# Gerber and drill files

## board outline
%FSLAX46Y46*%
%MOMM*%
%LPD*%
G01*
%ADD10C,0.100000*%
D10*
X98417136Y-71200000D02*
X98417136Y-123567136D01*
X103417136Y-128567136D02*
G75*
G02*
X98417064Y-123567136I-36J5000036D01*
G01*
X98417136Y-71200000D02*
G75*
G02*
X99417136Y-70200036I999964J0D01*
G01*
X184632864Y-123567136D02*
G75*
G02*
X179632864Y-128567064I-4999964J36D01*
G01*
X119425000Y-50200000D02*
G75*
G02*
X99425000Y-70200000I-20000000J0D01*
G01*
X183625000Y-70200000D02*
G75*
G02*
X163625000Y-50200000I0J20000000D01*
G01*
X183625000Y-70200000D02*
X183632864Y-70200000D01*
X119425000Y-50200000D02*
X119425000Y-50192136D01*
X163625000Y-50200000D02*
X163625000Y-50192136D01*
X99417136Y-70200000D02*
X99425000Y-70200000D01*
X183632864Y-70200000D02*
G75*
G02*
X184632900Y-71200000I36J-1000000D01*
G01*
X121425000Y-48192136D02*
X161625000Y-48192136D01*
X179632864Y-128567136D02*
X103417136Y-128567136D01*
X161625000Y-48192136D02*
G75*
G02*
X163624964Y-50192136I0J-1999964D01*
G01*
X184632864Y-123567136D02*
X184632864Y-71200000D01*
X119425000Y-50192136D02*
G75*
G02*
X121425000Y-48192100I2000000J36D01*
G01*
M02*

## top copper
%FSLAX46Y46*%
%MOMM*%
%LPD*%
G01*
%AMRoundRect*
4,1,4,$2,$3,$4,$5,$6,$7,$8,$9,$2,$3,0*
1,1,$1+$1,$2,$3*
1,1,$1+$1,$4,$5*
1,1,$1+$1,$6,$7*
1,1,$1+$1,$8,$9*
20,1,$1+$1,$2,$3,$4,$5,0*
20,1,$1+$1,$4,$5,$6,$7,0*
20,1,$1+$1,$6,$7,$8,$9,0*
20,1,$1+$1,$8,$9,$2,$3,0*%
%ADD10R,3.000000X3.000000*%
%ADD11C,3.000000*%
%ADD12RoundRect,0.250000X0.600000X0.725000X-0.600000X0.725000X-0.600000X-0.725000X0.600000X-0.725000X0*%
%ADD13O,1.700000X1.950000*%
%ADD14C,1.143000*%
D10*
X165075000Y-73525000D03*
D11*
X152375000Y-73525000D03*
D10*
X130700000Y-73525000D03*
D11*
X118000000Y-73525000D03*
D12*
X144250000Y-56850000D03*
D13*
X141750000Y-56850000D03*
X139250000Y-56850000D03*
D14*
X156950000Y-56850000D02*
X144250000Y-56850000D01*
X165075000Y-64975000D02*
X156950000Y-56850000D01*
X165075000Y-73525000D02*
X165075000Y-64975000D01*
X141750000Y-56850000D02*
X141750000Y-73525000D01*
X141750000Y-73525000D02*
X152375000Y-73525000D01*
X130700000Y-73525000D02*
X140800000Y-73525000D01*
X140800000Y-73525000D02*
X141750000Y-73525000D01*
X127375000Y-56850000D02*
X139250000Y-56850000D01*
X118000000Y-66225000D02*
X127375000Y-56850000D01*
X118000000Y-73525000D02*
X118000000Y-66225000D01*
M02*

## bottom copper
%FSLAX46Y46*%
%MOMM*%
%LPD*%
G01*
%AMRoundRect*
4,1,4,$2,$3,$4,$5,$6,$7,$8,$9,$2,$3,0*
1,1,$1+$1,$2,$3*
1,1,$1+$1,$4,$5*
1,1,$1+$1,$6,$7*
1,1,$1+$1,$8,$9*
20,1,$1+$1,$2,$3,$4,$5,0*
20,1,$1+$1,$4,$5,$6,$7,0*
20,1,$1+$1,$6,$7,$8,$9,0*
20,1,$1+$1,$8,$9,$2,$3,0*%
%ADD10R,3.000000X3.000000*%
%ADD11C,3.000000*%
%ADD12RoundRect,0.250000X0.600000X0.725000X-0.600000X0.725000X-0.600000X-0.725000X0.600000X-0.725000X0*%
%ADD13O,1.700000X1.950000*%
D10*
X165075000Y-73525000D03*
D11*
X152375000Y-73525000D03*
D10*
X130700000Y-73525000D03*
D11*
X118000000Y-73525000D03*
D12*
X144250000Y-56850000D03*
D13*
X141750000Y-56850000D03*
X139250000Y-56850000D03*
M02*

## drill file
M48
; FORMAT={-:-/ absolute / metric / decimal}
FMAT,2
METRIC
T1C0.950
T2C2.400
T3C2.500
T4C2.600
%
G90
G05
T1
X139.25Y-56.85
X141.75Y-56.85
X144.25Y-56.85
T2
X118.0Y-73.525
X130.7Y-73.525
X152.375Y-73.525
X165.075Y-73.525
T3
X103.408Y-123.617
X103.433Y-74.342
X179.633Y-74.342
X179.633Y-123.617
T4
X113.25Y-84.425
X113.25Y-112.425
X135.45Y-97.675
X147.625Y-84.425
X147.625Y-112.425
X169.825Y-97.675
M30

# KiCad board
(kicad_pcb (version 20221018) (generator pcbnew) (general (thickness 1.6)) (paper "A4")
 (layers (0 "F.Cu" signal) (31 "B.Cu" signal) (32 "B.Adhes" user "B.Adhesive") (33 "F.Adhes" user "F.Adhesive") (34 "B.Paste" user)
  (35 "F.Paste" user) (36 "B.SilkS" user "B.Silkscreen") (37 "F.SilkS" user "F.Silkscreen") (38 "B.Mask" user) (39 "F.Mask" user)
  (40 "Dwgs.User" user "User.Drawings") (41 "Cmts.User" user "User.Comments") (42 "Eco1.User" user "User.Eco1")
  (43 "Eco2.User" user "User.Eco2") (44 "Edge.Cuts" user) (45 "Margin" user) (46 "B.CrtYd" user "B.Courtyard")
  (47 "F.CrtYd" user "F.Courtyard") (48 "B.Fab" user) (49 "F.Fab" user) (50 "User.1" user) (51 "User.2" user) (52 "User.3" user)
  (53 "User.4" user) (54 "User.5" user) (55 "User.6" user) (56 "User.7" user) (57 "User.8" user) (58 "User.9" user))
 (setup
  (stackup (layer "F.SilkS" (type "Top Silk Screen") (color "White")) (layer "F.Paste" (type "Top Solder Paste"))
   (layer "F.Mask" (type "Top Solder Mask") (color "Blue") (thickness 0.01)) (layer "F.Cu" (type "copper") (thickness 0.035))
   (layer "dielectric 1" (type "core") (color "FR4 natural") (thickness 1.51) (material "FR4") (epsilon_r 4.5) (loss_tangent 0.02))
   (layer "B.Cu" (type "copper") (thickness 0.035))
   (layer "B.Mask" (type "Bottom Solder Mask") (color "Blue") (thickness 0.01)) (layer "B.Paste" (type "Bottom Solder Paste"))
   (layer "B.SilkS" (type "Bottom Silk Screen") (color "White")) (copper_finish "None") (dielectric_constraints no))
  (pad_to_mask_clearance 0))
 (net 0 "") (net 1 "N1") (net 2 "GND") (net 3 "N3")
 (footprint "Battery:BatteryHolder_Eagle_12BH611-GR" (layer "F.Cu") (at 165.075 73.525 90)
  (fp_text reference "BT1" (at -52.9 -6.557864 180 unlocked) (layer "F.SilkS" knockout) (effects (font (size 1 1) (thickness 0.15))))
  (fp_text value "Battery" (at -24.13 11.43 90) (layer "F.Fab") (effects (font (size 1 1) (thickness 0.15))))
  (pad "" np_thru_hole circle (at -38.9 -17.45 90) (size 2.6 2.6) (drill 2.6) (layers "*.Cu" "*.Mask"))
  (pad "" np_thru_hole circle (at -24.15 4.75 90) (size 2.6 2.6) (drill 2.6) (layers "*.Cu" "*.Mask"))
  (pad "" np_thru_hole circle (at -10.9 -17.45 90) (size 2.6 2.6) (drill 2.6) (layers "*.Cu" "*.Mask"))
  (pad "1" thru_hole rect (at 0 0 90) (size 3 3) (drill 2.4) (layers "*.Cu" "*.Mask") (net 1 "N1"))
  (pad "2" thru_hole circle (at 0 -12.7 90) (size 3 3) (drill 2.4) (layers "*.Cu" "*.Mask") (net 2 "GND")))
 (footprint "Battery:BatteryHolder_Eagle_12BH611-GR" (layer "F.Cu") (at 130.7 73.525 90)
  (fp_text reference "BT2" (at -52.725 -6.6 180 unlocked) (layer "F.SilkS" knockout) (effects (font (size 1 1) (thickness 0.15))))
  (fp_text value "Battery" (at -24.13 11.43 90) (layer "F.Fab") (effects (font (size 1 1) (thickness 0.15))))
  (pad "" np_thru_hole circle (at -38.9 -17.45 90) (size 2.6 2.6) (drill 2.6) (layers "*.Cu" "*.Mask"))
  (pad "" np_thru_hole circle (at -24.15 4.75 90) (size 2.6 2.6) (drill 2.6) (layers "*.Cu" "*.Mask"))
  (pad "" np_thru_hole circle (at -10.9 -17.45 90) (size 2.6 2.6) (drill 2.6) (layers "*.Cu" "*.Mask"))
  (pad "1" thru_hole rect (at 0 0 90) (size 3 3) (drill 2.4) (layers "*.Cu" "*.Mask") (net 2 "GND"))
  (pad "2" thru_hole circle (at 0 -12.7 90) (size 3 3) (drill 2.4) (layers "*.Cu" "*.Mask") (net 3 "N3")))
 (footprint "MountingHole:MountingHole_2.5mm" (layer "F.Cu") (at 103.432864 74.342136)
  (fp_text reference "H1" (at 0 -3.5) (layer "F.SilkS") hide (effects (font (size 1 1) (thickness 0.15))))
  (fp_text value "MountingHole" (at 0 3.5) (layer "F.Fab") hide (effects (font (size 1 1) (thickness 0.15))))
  (pad "" np_thru_hole circle (at 0 0) (size 2.5 2.5) (drill 2.5) (layers "*.Cu" "*.Mask")))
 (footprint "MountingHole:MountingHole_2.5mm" (layer "F.Cu") (at 103.407864 123.617136)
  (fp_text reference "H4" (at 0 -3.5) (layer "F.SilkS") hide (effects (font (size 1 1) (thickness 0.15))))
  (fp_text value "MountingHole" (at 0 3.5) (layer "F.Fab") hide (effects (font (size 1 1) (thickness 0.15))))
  (pad "" np_thru_hole circle (at 0 0) (size 2.5 2.5) (drill 2.5) (layers "*.Cu" "*.Mask")))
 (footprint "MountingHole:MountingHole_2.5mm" (layer "F.Cu") (at 179.632864 123.617136)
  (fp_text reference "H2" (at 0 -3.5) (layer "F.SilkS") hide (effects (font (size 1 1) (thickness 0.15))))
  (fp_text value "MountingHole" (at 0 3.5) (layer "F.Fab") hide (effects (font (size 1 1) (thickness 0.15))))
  (pad "" np_thru_hole circle (at 0 0) (size 2.5 2.5) (drill 2.5) (layers "*.Cu" "*.Mask")))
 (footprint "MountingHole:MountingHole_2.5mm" (layer "F.Cu") (at 179.632864 74.342136)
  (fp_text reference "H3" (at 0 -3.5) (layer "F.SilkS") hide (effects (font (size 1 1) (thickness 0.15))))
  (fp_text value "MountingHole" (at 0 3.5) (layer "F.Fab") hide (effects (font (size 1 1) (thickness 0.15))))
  (pad "" np_thru_hole circle (at 0 0) (size 2.5 2.5) (drill 2.5) (layers "*.Cu" "*.Mask")))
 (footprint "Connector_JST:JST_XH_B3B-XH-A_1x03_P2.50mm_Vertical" (layer "B.Cu") (at 144.25 56.85 180)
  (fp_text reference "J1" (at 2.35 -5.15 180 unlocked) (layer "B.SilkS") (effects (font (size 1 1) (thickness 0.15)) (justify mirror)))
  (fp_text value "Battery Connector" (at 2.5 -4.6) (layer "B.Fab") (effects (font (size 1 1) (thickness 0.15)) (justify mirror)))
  (pad "1" thru_hole roundrect (at 0 0 180) (size 1.7 1.95) (drill 0.95) (layers "*.Cu" "*.Mask") (roundrect_rratio 0.1470588235)
   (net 1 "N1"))
  (pad "2" thru_hole oval (at 2.5 0 180) (size 1.7 1.95) (drill 0.95) (layers "*.Cu" "*.Mask") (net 2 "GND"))
  (pad "3" thru_hole oval (at 5 0 180) (size 1.7 1.95) (drill 0.95) (layers "*.Cu" "*.Mask") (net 3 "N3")))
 (gr_line (start 98.417136 71.2) (end 98.417136 123.567136) (stroke (width 0.1) (type default)) (layer "Edge.Cuts"))
 (gr_arc (start 103.417136 128.567136) (mid 99.881602 127.10267) (end 98.417136 123.567136) (stroke (width 0.1) (type default))
  (layer "Edge.Cuts"))
 (gr_arc (start 98.417136 71.2) (mid 98.710029 70.492893) (end 99.417136 70.2) (stroke (width 0.1) (type default)) (layer "Edge.Cuts"))
 (gr_arc (start 184.632864 123.567136) (mid 183.168398 127.10267) (end 179.632864 128.567136) (stroke (width 0.1) (type default))
  (layer "Edge.Cuts"))
 (gr_arc (start 119.425 50.2) (mid 113.567136 64.342136) (end 99.425 70.2) (stroke (width 0.1) (type default)) (layer "Edge.Cuts"))
 (gr_arc (start 183.625 70.2) (mid 169.482864 64.342136) (end 163.625 50.2) (stroke (width 0.1) (type default)) (layer "Edge.Cuts"))
 (gr_line (start 183.625 70.2) (end 183.632864 70.2) (stroke (width 0.1) (type default)) (layer "Edge.Cuts"))
 (gr_line (start 119.425 50.2) (end 119.425 50.192136) (stroke (width 0.1) (type default)) (layer "Edge.Cuts"))
 (gr_line (start 163.625 50.2) (end 163.625 50.192136) (stroke (width 0.1) (type default)) (layer "Edge.Cuts"))
 (gr_line (start 99.417136 70.2) (end 99.425 70.2) (stroke (width 0.1) (type default)) (layer "Edge.Cuts"))
 (gr_arc (start 183.632864 70.2) (mid 184.339971 70.492893) (end 184.632864 71.2) (stroke (width 0.1) (type default)) (layer "Edge.Cuts"))
 (gr_line (start 121.425 48.192136) (end 161.625 48.192136) (stroke (width 0.1) (type default)) (layer "Edge.Cuts"))
 (gr_line (start 179.632864 128.567136) (end 103.417136 128.567136) (stroke (width 0.1) (type default)) (layer "Edge.Cuts"))
 (gr_arc (start 161.625 48.192136) (mid 163.039214 48.777922) (end 163.625 50.192136) (stroke (width 0.1) (type default))
  (layer "Edge.Cuts"))
 (gr_line (start 184.632864 123.567136) (end 184.632864 71.2) (stroke (width 0.1) (type default)) (layer "Edge.Cuts"))
 (gr_arc (start 119.425 50.192136) (mid 120.010786 48.777922) (end 121.425 48.192136) (stroke (width 0.1) (type default))
  (layer "Edge.Cuts"))
 (segment (start 156.95 56.85) (end 144.25 56.85) (width 1.143) (layer "F.Cu") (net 1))
 (segment (start 165.075 64.975) (end 156.95 56.85) (width 1.143) (layer "F.Cu") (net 1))
 (segment (start 165.075 73.525) (end 165.075 64.975) (width 1.143) (layer "F.Cu") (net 1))
 (segment (start 141.75 56.85) (end 141.75 73.525) (width 1.143) (layer "F.Cu") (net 2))
 (segment (start 141.75 73.525) (end 152.375 73.525) (width 1.143) (layer "F.Cu") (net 2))
 (segment (start 130.7 73.525) (end 140.8 73.525) (width 1.143) (layer "F.Cu") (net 2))
 (segment (start 140.8 73.525) (end 141.75 73.525) (width 1.143) (layer "F.Cu") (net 2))
 (segment (start 127.375 56.85) (end 139.25 56.85) (width 1.143) (layer "F.Cu") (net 3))
 (segment (start 118 66.225) (end 127.375 56.85) (width 1.143) (layer "F.Cu") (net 3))
 (segment (start 118 73.525) (end 118 66.225) (width 1.143) (layer "F.Cu") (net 3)))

